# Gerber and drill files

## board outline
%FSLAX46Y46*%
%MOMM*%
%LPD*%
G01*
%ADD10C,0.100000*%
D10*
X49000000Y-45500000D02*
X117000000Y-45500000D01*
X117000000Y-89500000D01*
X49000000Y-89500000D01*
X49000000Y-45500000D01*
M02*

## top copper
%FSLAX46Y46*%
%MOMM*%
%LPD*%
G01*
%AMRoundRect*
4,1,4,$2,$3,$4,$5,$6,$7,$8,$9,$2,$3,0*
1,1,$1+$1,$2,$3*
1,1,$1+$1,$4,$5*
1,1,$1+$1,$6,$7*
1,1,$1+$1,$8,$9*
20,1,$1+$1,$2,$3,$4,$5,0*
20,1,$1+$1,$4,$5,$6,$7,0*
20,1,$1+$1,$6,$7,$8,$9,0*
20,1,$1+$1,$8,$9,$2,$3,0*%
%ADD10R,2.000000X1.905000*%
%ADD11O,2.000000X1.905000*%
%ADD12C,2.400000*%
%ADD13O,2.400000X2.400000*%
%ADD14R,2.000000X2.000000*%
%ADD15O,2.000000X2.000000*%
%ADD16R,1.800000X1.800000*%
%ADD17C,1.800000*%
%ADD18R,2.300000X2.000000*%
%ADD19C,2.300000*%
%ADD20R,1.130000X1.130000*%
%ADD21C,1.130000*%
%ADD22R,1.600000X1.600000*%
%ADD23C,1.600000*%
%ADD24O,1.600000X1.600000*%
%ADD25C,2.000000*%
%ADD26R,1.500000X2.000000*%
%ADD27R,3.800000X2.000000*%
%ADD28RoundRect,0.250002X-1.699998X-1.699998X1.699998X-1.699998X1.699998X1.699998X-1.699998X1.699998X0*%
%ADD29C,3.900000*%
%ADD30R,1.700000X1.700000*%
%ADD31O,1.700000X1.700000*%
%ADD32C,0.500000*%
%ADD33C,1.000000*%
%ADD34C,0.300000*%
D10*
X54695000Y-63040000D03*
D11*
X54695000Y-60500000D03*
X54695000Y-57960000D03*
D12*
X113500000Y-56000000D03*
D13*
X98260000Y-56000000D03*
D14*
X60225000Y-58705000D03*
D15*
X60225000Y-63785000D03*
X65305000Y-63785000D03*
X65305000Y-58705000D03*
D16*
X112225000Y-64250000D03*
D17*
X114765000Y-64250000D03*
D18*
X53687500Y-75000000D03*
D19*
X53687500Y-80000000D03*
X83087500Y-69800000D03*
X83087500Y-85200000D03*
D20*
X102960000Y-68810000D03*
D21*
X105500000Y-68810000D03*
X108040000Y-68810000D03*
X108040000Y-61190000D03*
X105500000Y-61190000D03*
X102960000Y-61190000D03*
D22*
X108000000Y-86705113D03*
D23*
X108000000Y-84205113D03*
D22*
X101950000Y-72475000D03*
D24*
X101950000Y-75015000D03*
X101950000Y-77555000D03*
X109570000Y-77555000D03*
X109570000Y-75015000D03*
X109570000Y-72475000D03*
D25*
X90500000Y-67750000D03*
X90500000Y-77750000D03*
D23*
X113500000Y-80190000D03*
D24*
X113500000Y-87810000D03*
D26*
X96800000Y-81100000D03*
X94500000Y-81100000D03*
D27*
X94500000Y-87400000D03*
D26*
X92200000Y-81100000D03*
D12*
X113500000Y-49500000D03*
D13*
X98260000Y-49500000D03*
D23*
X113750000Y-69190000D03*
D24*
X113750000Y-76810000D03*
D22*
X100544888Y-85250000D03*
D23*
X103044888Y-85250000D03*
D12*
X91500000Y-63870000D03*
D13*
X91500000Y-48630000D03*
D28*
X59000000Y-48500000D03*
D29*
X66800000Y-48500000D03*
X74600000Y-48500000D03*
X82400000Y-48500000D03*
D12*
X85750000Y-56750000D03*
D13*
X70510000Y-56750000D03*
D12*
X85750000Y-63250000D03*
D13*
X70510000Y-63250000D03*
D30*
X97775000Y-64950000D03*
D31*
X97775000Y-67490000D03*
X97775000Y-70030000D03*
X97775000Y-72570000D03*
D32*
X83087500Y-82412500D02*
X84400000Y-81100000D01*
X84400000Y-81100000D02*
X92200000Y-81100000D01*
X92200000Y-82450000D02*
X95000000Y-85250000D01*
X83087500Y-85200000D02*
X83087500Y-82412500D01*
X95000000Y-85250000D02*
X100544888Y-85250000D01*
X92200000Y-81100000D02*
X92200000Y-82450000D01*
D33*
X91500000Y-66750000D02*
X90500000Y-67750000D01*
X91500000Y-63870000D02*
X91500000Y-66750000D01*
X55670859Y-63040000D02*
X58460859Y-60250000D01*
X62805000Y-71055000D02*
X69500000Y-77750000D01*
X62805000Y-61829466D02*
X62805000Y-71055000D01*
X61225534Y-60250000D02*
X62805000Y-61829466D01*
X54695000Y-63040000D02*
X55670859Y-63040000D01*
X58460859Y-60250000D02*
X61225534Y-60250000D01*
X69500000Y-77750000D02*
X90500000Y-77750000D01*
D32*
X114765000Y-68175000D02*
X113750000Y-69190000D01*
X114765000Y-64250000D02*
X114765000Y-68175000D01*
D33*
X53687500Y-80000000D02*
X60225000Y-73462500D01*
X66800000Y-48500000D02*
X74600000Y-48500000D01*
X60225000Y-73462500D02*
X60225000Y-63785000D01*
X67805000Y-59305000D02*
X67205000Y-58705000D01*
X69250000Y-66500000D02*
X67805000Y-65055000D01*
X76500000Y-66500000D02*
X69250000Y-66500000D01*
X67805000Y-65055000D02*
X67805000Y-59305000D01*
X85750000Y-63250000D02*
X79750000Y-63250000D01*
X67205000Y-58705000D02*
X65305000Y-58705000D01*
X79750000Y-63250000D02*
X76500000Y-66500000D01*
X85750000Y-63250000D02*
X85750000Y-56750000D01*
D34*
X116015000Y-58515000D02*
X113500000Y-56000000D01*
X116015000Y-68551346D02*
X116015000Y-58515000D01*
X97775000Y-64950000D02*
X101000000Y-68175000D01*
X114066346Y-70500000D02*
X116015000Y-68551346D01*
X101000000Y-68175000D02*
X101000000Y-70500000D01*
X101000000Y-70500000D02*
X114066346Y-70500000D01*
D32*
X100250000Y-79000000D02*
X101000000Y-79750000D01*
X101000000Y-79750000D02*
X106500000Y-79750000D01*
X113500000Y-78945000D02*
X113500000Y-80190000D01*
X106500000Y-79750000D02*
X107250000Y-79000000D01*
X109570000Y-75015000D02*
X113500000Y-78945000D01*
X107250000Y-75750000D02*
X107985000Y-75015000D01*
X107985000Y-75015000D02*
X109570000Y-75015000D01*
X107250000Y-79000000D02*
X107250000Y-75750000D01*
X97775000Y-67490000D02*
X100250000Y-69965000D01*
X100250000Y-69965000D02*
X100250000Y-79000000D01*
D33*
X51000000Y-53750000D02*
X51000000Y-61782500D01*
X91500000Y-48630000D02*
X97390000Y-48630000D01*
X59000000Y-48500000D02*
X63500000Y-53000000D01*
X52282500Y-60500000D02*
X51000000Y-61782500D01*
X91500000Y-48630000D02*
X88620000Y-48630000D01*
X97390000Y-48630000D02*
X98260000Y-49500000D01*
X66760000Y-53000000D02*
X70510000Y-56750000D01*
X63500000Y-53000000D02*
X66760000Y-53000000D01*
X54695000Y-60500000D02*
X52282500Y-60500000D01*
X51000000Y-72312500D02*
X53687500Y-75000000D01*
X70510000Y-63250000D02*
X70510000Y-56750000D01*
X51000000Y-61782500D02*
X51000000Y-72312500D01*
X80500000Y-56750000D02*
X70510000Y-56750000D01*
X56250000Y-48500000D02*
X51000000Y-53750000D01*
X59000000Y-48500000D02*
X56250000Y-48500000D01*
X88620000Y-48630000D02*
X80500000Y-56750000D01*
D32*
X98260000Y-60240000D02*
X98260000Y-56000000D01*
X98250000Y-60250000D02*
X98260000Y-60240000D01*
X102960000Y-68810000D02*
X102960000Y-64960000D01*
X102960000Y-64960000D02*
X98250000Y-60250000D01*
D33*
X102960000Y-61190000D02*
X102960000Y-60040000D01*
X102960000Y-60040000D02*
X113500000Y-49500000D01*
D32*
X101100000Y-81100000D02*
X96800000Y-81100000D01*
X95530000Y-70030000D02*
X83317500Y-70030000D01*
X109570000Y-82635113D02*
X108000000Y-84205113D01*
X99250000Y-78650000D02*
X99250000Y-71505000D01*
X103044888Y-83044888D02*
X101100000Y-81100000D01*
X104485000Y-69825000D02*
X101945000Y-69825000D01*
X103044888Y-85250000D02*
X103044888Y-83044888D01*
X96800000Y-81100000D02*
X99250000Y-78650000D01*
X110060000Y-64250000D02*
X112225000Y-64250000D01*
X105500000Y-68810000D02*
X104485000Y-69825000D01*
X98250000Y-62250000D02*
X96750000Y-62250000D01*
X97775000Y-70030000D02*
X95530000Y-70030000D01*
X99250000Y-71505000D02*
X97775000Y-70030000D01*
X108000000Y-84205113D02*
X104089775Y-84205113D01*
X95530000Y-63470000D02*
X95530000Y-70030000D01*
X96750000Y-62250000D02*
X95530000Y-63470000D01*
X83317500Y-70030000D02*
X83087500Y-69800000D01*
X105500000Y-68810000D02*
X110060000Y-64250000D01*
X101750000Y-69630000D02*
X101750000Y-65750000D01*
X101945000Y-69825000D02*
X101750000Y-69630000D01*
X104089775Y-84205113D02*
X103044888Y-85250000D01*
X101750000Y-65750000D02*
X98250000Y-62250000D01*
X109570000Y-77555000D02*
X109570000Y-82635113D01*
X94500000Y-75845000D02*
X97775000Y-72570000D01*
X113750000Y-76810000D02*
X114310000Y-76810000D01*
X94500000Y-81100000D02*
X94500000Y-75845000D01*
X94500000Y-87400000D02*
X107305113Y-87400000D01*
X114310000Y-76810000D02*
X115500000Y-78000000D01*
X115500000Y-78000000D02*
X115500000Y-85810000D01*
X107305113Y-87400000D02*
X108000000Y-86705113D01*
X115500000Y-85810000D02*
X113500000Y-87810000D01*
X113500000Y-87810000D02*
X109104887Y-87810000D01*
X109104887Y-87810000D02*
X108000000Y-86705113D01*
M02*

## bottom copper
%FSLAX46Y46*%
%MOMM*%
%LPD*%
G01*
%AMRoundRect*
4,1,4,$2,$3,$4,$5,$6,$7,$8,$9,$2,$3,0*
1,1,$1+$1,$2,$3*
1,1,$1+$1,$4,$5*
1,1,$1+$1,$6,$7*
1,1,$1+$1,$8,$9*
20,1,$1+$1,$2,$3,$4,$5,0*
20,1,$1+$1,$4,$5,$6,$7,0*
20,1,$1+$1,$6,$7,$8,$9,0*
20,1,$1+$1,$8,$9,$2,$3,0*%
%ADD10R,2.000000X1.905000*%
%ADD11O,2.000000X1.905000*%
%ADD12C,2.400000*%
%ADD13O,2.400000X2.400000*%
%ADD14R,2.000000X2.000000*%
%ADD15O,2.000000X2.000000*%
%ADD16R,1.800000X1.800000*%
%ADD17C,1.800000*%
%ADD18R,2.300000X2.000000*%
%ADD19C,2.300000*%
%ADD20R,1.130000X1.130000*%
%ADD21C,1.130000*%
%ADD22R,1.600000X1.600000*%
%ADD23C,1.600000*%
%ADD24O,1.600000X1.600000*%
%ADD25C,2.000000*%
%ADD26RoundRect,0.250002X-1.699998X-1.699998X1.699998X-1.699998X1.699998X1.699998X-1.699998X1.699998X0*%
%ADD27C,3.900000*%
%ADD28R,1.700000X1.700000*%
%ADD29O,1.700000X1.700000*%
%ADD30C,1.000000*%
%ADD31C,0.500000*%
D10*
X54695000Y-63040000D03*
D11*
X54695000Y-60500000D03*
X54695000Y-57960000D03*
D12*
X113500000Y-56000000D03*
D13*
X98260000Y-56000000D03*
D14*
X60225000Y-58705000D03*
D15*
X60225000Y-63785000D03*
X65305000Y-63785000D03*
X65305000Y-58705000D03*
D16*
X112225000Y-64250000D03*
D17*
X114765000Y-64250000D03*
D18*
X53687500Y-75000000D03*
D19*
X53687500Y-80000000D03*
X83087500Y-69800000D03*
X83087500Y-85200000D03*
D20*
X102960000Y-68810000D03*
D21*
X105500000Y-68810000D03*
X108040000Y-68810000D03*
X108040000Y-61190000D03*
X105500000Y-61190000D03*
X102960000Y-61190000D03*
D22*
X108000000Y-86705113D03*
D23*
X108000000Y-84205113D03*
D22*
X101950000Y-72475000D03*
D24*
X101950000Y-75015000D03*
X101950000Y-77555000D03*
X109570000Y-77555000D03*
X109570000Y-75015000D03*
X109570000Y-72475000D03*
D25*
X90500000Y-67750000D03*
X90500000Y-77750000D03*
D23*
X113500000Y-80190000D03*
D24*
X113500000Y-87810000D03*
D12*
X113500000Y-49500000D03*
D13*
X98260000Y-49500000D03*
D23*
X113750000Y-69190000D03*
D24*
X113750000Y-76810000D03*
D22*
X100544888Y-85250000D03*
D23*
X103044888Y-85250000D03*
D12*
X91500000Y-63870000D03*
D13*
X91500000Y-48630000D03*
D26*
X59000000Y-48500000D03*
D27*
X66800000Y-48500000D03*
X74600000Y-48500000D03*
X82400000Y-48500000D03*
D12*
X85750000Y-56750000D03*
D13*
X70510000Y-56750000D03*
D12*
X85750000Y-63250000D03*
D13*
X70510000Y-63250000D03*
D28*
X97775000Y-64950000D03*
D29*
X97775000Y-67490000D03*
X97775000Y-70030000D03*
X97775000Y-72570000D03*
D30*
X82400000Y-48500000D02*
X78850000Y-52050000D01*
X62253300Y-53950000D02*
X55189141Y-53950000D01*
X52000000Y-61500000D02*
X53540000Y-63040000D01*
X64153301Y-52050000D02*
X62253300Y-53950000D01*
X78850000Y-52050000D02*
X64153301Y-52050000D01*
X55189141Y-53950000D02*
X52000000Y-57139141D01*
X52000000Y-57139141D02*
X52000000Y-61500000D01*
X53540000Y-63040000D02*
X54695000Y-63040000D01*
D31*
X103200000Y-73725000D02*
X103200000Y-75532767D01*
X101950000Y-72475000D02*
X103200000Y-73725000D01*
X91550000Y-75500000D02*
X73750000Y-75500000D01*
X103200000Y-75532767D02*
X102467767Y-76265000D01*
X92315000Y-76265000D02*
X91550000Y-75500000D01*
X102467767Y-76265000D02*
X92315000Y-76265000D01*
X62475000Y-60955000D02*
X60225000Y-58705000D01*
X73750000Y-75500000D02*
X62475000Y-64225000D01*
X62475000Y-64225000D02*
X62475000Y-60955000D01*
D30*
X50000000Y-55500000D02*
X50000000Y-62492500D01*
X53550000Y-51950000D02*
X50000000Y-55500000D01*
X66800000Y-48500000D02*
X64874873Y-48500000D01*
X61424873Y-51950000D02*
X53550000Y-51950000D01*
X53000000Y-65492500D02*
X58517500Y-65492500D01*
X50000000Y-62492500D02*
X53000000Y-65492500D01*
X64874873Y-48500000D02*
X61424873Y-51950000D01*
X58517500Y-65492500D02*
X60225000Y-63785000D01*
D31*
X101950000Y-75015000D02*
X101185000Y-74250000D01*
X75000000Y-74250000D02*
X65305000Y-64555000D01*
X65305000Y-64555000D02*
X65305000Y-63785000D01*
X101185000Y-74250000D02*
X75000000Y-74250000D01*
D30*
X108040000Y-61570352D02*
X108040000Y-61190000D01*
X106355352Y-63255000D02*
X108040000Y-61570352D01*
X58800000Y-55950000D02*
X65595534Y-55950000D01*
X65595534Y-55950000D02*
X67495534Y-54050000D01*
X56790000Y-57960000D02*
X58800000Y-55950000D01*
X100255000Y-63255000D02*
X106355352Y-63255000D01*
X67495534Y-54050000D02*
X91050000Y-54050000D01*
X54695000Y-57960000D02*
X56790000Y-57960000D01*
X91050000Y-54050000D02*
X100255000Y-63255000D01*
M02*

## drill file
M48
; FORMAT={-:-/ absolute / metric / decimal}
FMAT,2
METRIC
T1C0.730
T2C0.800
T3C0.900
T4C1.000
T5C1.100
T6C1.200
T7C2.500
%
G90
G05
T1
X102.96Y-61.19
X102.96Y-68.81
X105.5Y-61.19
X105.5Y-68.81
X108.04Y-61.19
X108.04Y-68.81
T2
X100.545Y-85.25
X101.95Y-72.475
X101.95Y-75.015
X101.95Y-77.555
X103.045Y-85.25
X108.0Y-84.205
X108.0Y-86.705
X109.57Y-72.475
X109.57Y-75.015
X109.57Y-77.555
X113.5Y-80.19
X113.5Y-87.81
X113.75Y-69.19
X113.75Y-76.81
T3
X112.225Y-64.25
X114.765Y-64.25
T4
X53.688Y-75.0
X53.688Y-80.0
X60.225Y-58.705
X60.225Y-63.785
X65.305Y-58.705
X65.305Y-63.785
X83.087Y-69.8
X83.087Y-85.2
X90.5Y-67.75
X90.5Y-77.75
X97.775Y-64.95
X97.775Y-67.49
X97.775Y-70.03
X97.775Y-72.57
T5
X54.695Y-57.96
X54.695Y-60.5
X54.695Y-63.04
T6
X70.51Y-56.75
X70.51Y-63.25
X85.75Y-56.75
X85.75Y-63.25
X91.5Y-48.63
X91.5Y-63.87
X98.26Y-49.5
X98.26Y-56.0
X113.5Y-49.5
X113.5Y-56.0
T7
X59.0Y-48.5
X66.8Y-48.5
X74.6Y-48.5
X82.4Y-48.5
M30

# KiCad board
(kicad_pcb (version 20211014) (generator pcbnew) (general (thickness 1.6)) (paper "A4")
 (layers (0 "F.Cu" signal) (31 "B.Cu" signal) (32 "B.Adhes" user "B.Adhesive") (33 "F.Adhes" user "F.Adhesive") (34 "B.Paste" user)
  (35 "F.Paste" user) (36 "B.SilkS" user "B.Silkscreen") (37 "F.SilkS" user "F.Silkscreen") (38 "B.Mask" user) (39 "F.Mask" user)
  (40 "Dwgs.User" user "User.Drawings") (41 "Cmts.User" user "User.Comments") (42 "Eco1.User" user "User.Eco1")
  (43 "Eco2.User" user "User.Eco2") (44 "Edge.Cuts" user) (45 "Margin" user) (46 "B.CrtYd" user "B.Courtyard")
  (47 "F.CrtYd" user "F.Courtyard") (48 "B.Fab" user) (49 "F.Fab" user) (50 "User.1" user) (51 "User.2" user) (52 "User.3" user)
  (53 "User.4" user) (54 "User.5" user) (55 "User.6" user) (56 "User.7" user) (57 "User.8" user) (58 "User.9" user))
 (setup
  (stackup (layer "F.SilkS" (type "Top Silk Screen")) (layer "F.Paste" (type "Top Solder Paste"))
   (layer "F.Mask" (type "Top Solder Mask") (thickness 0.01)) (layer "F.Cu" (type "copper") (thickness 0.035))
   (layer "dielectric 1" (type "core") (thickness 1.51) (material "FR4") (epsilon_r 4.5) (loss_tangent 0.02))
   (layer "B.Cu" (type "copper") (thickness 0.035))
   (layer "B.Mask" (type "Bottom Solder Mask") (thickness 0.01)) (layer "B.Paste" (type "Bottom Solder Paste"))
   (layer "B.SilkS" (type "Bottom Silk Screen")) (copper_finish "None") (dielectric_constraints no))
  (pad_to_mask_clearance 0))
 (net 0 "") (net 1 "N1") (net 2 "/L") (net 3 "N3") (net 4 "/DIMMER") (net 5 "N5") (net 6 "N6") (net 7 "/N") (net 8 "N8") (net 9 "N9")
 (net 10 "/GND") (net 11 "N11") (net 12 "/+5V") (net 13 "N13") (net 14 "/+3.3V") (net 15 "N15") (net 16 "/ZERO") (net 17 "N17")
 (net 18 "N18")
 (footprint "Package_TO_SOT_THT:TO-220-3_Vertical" (layer "F.Cu") (at 54.695 63.04 90)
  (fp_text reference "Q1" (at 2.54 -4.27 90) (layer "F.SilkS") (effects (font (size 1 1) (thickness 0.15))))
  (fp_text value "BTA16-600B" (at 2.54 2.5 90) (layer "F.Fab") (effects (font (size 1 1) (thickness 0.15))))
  (pad "1" thru_hole rect (at 0 0 90) (size 1.905 2) (drill 1.1) (layers *.Cu *.Mask) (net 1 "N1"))
  (pad "2" thru_hole oval (at 2.54 0 90) (size 1.905 2) (drill 1.1) (layers *.Cu *.Mask) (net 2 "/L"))
  (pad "3" thru_hole oval (at 5.08 0 90) (size 1.905 2) (drill 1.1) (layers *.Cu *.Mask) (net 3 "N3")))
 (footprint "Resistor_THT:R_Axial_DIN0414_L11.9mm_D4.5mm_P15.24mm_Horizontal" (layer "F.Cu") (at 113.5 56 180)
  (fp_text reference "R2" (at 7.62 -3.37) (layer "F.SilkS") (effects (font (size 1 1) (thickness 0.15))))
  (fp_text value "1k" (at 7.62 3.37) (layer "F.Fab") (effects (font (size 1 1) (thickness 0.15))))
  (pad "1" thru_hole circle (at 0 0 180) (size 2.4 2.4) (drill 1.2) (layers *.Cu *.Mask) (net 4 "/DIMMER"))
  (pad "2" thru_hole oval (at 15.24 0 180) (size 2.4 2.4) (drill 1.2) (layers *.Cu *.Mask) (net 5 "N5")))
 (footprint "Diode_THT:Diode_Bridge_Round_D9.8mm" (layer "F.Cu") (at 60.225 58.705)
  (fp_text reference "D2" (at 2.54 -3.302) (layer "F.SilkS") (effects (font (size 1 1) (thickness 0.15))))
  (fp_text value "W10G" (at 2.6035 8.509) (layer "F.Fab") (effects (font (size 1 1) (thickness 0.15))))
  (pad "1" thru_hole rect (at 0 0) (size 2 2) (drill 1) (layers *.Cu *.Mask) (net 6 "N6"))
  (pad "2" thru_hole oval (at 0 5.08) (size 2 2) (drill 1) (layers *.Cu *.Mask) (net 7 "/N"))
  (pad "3" thru_hole oval (at 5.08 5.08) (size 2 2) (drill 1) (layers *.Cu *.Mask) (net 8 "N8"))
  (pad "4" thru_hole oval (at 5.08 0) (size 2 2) (drill 1) (layers *.Cu *.Mask) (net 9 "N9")))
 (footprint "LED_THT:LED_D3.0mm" (layer "F.Cu") (at 112.225 64.25)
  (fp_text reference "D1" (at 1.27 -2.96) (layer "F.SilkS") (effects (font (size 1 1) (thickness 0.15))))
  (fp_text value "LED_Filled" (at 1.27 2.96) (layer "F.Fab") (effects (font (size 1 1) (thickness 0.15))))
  (pad "1" thru_hole rect (at 0 0) (size 1.8 1.8) (drill 0.9) (layers *.Cu *.Mask) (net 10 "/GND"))
  (pad "2" thru_hole circle (at 2.54 0) (size 1.8 1.8) (drill 0.9) (layers *.Cu *.Mask) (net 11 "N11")))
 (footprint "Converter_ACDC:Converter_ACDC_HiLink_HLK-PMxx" (layer "F.Cu") (at 53.6875 75)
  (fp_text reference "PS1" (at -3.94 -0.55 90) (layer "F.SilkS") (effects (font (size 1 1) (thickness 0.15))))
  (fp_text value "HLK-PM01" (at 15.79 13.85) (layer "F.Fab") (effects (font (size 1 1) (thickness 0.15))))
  (pad "1" thru_hole rect (at 0 0) (size 2.3 2) (drill 1) (layers *.Cu *.Mask) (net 2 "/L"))
  (pad "2" thru_hole circle (at 0 5) (size 2.3 2.3) (drill 1) (layers *.Cu *.Mask) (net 7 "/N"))
  (pad "3" thru_hole circle (at 29.4 -5.2) (size 2.3 2.3) (drill 1) (layers *.Cu *.Mask) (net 10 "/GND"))
  (pad "4" thru_hole circle (at 29.4 10.2) (size 2.3 2.3) (drill 1) (layers *.Cu *.Mask) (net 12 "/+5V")))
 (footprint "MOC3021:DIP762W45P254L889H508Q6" (layer "F.Cu") (at 105.5 65 90)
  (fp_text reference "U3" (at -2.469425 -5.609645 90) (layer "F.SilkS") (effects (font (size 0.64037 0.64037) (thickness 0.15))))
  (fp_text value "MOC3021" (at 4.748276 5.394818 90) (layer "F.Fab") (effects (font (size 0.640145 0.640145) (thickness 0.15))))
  (pad "1" thru_hole rect locked (at -3.81 -2.54 90) (size 1.13 1.13) (drill 0.73) (layers *.Cu *.Mask) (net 5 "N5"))
  (pad "2" thru_hole circle locked (at -3.81 0 90) (size 1.13 1.13) (drill 0.73) (layers *.Cu *.Mask) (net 10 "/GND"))
  (pad "3" thru_hole circle locked (at -3.81 2.54 90) (size 1.13 1.13) (drill 0.73) (layers *.Cu *.Mask))
  (pad "4" thru_hole circle locked (at 3.81 2.54 90) (size 1.13 1.13) (drill 0.73) (layers *.Cu *.Mask) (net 3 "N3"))
  (pad "5" thru_hole circle locked (at 3.81 0 90) (size 1.13 1.13) (drill 0.73) (layers *.Cu *.Mask))
  (pad "6" thru_hole circle locked (at 3.81 -2.54 90) (size 1.13 1.13) (drill 0.73) (layers *.Cu *.Mask) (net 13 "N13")))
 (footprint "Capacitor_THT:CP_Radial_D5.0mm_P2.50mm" (layer "F.Cu") (at 108 86.705113 90)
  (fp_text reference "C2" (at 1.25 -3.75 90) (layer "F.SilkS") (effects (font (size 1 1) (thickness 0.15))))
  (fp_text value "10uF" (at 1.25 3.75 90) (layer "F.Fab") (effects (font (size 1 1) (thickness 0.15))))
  (pad "1" thru_hole rect (at 0 0 90) (size 1.6 1.6) (drill 0.8) (layers *.Cu *.Mask) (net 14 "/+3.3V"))
  (pad "2" thru_hole circle (at 2.5 0 90) (size 1.6 1.6) (drill 0.8) (layers *.Cu *.Mask) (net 10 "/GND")))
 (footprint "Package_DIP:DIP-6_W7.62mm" (layer "F.Cu") (at 101.95 72.475)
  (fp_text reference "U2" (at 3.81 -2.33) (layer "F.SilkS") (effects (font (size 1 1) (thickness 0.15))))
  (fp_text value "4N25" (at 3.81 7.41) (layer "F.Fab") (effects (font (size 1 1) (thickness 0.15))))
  (pad "1" thru_hole rect (at 0 0) (size 1.6 1.6) (drill 0.8) (layers *.Cu *.Mask) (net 6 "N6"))
  (pad "2" thru_hole oval (at 0 2.54) (size 1.6 1.6) (drill 0.8) (layers *.Cu *.Mask) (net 8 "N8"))
  (pad "3" thru_hole oval (at 0 5.08) (size 1.6 1.6) (drill 0.8) (layers *.Cu *.Mask) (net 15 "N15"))
  (pad "4" thru_hole oval (at 7.62 5.08) (size 1.6 1.6) (drill 0.8) (layers *.Cu *.Mask) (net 10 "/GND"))
  (pad "5" thru_hole oval (at 7.62 2.54) (size 1.6 1.6) (drill 0.8) (layers *.Cu *.Mask) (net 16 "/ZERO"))
  (pad "6" thru_hole oval (at 7.62 0) (size 1.6 1.6) (drill 0.8) (layers *.Cu *.Mask) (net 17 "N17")))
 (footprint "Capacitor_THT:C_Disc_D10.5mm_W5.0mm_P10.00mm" (layer "F.Cu") (at 90.5 67.75 -90)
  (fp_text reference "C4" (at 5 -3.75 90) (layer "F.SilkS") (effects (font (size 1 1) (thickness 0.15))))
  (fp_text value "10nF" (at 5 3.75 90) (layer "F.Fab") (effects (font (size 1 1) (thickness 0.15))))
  (pad "1" thru_hole circle (at 0 0 270) (size 2 2) (drill 1) (layers *.Cu *.Mask) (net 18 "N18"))
  (pad "2" thru_hole circle (at 10 0 270) (size 2 2) (drill 1) (layers *.Cu *.Mask) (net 1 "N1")))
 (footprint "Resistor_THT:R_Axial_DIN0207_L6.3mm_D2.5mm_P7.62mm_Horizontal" (layer "F.Cu") (at 113.5 80.19 -90)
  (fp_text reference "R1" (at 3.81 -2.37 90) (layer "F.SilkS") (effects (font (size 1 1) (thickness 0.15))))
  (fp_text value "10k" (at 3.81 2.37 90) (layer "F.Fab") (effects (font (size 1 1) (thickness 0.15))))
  (pad "1" thru_hole circle (at 0 0 270) (size 1.6 1.6) (drill 0.8) (layers *.Cu *.Mask) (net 16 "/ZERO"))
  (pad "2" thru_hole oval (at 7.62 0 270) (size 1.6 1.6) (drill 0.8) (layers *.Cu *.Mask) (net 14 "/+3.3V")))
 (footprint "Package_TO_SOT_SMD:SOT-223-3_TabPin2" (layer "F.Cu") (at 94.5 84.25 -90)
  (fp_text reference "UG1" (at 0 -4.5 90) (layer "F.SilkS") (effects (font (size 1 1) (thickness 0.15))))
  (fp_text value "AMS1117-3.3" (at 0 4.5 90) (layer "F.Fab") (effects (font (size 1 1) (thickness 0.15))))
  (pad "1" smd rect (at -3.15 -2.3 270) (size 2 1.5) (layers "F.Cu" "F.Paste" "F.Mask") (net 10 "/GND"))
  (pad "2" smd rect (at -3.15 0 270) (size 2 1.5) (layers "F.Cu" "F.Paste" "F.Mask") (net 14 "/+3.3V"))
  (pad "2" smd rect (at 3.15 0 270) (size 2 3.8) (layers "F.Cu" "F.Paste" "F.Mask") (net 14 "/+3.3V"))
  (pad "3" smd rect (at -3.15 2.3 270) (size 2 1.5) (layers "F.Cu" "F.Paste" "F.Mask") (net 12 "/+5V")))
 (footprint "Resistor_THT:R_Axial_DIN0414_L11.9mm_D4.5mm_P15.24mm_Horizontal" (layer "F.Cu") (at 113.5 49.5 180)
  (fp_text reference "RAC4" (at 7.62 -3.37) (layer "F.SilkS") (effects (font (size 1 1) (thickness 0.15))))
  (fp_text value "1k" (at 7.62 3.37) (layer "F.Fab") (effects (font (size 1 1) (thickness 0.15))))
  (pad "1" thru_hole circle (at 0 0 180) (size 2.4 2.4) (drill 1.2) (layers *.Cu *.Mask) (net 13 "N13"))
  (pad "2" thru_hole oval (at 15.24 0 180) (size 2.4 2.4) (drill 1.2) (layers *.Cu *.Mask) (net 2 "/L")))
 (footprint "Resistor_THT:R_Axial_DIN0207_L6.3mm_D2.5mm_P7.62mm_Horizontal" (layer "F.Cu") (at 113.75 69.19 -90)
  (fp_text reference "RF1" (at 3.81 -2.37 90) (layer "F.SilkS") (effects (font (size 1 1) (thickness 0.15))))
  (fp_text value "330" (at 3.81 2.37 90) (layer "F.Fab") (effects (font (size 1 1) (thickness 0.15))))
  (pad "1" thru_hole circle (at 0 0 270) (size 1.6 1.6) (drill 0.8) (layers *.Cu *.Mask) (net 11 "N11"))
  (pad "2" thru_hole oval (at 7.62 0 270) (size 1.6 1.6) (drill 0.8) (layers *.Cu *.Mask) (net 14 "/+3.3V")))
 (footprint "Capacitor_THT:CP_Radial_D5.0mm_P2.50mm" (layer "F.Cu") (at 100.544888 85.25)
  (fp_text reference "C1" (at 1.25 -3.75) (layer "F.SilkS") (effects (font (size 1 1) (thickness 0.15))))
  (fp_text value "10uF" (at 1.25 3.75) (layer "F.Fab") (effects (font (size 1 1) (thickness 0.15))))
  (pad "1" thru_hole rect (at 0 0) (size 1.6 1.6) (drill 0.8) (layers *.Cu *.Mask) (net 12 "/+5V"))
  (pad "2" thru_hole circle (at 2.5 0) (size 1.6 1.6) (drill 0.8) (layers *.Cu *.Mask) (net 10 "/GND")))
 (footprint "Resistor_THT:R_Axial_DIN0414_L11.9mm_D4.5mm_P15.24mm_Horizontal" (layer "F.Cu") (at 91.5 63.87 90)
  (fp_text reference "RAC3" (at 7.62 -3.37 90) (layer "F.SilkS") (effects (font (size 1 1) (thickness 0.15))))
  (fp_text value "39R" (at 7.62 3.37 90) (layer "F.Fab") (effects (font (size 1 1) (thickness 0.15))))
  (pad "1" thru_hole circle (at 0 0 90) (size 2.4 2.4) (drill 1.2) (layers *.Cu *.Mask) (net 18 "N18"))
  (pad "2" thru_hole oval (at 15.24 0 90) (size 2.4 2.4) (drill 1.2) (layers *.Cu *.Mask) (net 2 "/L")))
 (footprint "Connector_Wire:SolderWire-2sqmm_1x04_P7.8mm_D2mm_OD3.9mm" (layer "F.Cu") (at 59 48.5)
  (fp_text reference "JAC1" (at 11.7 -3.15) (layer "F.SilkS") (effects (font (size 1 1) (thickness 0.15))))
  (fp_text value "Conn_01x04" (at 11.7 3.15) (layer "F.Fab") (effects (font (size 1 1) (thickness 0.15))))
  (pad "1" thru_hole roundrect (at 0 0) (size 3.9 3.9) (drill 2.5) (layers *.Cu *.Mask) (roundrect_rratio 0.064103) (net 2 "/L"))
  (pad "2" thru_hole circle (at 7.8 0) (size 3.9 3.9) (drill 2.5) (layers *.Cu *.Mask) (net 7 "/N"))
  (pad "3" thru_hole circle (at 15.6 0) (size 3.9 3.9) (drill 2.5) (layers *.Cu *.Mask) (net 7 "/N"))
  (pad "4" thru_hole circle (at 23.4 0) (size 3.9 3.9) (drill 2.5) (layers *.Cu *.Mask) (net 1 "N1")))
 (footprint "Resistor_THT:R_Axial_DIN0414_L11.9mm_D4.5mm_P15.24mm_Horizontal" (layer "F.Cu") (at 85.75 56.75 180)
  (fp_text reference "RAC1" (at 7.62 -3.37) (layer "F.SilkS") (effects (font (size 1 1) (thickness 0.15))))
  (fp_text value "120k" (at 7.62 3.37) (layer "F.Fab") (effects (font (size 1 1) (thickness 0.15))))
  (pad "1" thru_hole circle (at 0 0 180) (size 2.4 2.4) (drill 1.2) (layers *.Cu *.Mask) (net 9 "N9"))
  (pad "2" thru_hole oval (at 15.24 0 180) (size 2.4 2.4) (drill 1.2) (layers *.Cu *.Mask) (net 2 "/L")))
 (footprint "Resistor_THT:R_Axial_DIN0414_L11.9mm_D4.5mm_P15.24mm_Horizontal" (layer "F.Cu") (at 85.75 63.25 180)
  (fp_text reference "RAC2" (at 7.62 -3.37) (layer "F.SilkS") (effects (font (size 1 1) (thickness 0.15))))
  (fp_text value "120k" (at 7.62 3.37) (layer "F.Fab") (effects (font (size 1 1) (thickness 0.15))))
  (pad "1" thru_hole circle (at 0 0 180) (size 2.4 2.4) (drill 1.2) (layers *.Cu *.Mask) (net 9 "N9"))
  (pad "2" thru_hole oval (at 15.24 0 180) (size 2.4 2.4) (drill 1.2) (layers *.Cu *.Mask) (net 2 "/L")))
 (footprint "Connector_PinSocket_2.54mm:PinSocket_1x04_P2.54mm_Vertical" (layer "F.Cu") (at 97.775 64.95)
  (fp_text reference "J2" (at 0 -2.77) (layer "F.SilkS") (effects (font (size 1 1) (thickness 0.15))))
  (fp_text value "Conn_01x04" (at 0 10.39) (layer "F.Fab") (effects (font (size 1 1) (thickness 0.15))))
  (pad "1" thru_hole rect (at 0 0) (size 1.7 1.7) (drill 1) (layers *.Cu *.Mask) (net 4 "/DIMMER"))
  (pad "2" thru_hole oval (at 0 2.54) (size 1.7 1.7) (drill 1) (layers *.Cu *.Mask) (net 16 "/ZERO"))
  (pad "3" thru_hole oval (at 0 5.08) (size 1.7 1.7) (drill 1) (layers *.Cu *.Mask) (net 10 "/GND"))
  (pad "4" thru_hole oval (at 0 7.62) (size 1.7 1.7) (drill 1) (layers *.Cu *.Mask) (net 14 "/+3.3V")))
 (gr_rect (start 49 45.5) (end 117 89.5) (layer "Edge.Cuts") (width 0.1) (fill none))
 (segment (start 83.0875 82.4125) (end 84.4 81.1) (width 0.5) (layer "F.Cu") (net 12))
 (segment (start 84.4 81.1) (end 92.2 81.1) (width 0.5) (layer "F.Cu") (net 12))
 (segment (start 92.2 82.45) (end 95 85.25) (width 0.5) (layer "F.Cu") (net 12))
 (segment (start 83.0875 85.2) (end 83.0875 82.4125) (width 0.5) (layer "F.Cu") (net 12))
 (segment (start 95 85.25) (end 100.544888 85.25) (width 0.5) (layer "F.Cu") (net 12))
 (segment (start 92.2 81.1) (end 92.2 82.45) (width 0.5) (layer "F.Cu") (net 12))
 (segment (start 91.5 66.75) (end 90.5 67.75) (width 1) (layer "F.Cu") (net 18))
 (segment (start 91.5 63.87) (end 91.5 66.75) (width 1) (layer "F.Cu") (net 18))
 (segment (start 55.670859 63.04) (end 58.460859 60.25) (width 1) (layer "F.Cu") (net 1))
 (segment (start 62.805 71.055) (end 69.5 77.75) (width 1) (layer "F.Cu") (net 1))
 (segment (start 62.805 61.829466) (end 62.805 71.055) (width 1) (layer "F.Cu") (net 1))
 (segment (start 61.225534 60.25) (end 62.805 61.829466) (width 1) (layer "F.Cu") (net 1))
 (segment (start 54.695 63.04) (end 55.670859 63.04) (width 1) (layer "F.Cu") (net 1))
 (segment (start 58.460859 60.25) (end 61.225534 60.25) (width 1) (layer "F.Cu") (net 1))
 (segment (start 69.5 77.75) (end 90.5 77.75) (width 1) (layer "F.Cu") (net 1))
 (segment (start 82.4 48.5) (end 78.85 52.05) (width 1) (layer "B.Cu") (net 1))
 (segment (start 62.2533 53.95) (end 55.189141 53.95) (width 1) (layer "B.Cu") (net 1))
 (segment (start 52 61.5) (end 53.54 63.04) (width 1) (layer "B.Cu") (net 1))
 (segment (start 64.153301 52.05) (end 62.2533 53.95) (width 1) (layer "B.Cu") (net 1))
 (segment (start 78.85 52.05) (end 64.153301 52.05) (width 1) (layer "B.Cu") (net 1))
 (segment (start 55.189141 53.95) (end 52 57.139141) (width 1) (layer "B.Cu") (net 1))
 (segment (start 52 57.139141) (end 52 61.5) (width 1) (layer "B.Cu") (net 1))
 (segment (start 53.54 63.04) (end 54.695 63.04) (width 1) (layer "B.Cu") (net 1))
 (segment (start 114.765 68.175) (end 113.75 69.19) (width 0.5) (layer "F.Cu") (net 11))
 (segment (start 114.765 64.25) (end 114.765 68.175) (width 0.5) (layer "F.Cu") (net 11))
 (segment (start 103.2 73.725) (end 103.2 75.532767) (width 0.5) (layer "B.Cu") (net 6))
 (segment (start 101.95 72.475) (end 103.2 73.725) (width 0.5) (layer "B.Cu") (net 6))
 (segment (start 91.55 75.5) (end 73.75 75.5) (width 0.5) (layer "B.Cu") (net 6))
 (segment (start 103.2 75.532767) (end 102.467767 76.265) (width 0.5) (layer "B.Cu") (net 6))
 (segment (start 92.315 76.265) (end 91.55 75.5) (width 0.5) (layer "B.Cu") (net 6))
 (segment (start 102.467767 76.265) (end 92.315 76.265) (width 0.5) (layer "B.Cu") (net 6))
 (segment (start 62.475 60.955) (end 60.225 58.705) (width 0.5) (layer "B.Cu") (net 6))
 (segment (start 73.75 75.5) (end 62.475 64.225) (width 0.5) (layer "B.Cu") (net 6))
 (segment (start 62.475 64.225) (end 62.475 60.955) (width 0.5) (layer "B.Cu") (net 6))
 (segment (start 53.6875 80) (end 60.225 73.4625) (width 1) (layer "F.Cu") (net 7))
 (segment (start 66.8 48.5) (end 74.6 48.5) (width 1) (layer "F.Cu") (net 7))
 (segment (start 60.225 73.4625) (end 60.225 63.785) (width 1) (layer "F.Cu") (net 7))
 (segment (start 50 55.5) (end 50 62.4925) (width 1) (layer "B.Cu") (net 7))
 (segment (start 53.55 51.95) (end 50 55.5) (width 1) (layer "B.Cu") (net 7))
 (segment (start 66.8 48.5) (end 64.874873 48.5) (width 1) (layer "B.Cu") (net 7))
 (segment (start 61.424873 51.95) (end 53.55 51.95) (width 1) (layer "B.Cu") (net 7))
 (segment (start 53 65.4925) (end 58.5175 65.4925) (width 1) (layer "B.Cu") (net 7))
 (segment (start 50 62.4925) (end 53 65.4925) (width 1) (layer "B.Cu") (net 7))
 (segment (start 64.874873 48.5) (end 61.424873 51.95) (width 1) (layer "B.Cu") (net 7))
 (segment (start 58.5175 65.4925) (end 60.225 63.785) (width 1) (layer "B.Cu") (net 7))
 (segment (start 101.95 75.015) (end 101.185 74.25) (width 0.5) (layer "B.Cu") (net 8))
 (segment (start 75 74.25) (end 65.305 64.555) (width 0.5) (layer "B.Cu") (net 8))
 (segment (start 65.305 64.555) (end 65.305 63.785) (width 0.5) (layer "B.Cu") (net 8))
 (segment (start 101.185 74.25) (end 75 74.25) (width 0.5) (layer "B.Cu") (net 8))
 (segment (start 67.805 59.305) (end 67.205 58.705) (width 1) (layer "F.Cu") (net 9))
 (segment (start 69.25 66.5) (end 67.805 65.055) (width 1) (layer "F.Cu") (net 9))
 (segment (start 76.5 66.5) (end 69.25 66.5) (width 1) (layer "F.Cu") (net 9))
 (segment (start 67.805 65.055) (end 67.805 59.305) (width 1) (layer "F.Cu") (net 9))
 (segment (start 85.75 63.25) (end 79.75 63.25) (width 1) (layer "F.Cu") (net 9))
 (segment (start 67.205 58.705) (end 65.305 58.705) (width 1) (layer "F.Cu") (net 9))
 (segment (start 79.75 63.25) (end 76.5 66.5) (width 1) (layer "F.Cu") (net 9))
 (segment (start 85.75 63.25) (end 85.75 56.75) (width 1) (layer "F.Cu") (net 9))
 (segment (start 116.015 58.515) (end 113.5 56) (width 0.3) (layer "F.Cu") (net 4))
 (segment (start 116.015 68.551346) (end 116.015 58.515) (width 0.3) (layer "F.Cu") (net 4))
 (segment (start 97.775 64.95) (end 101 68.175) (width 0.3) (layer "F.Cu") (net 4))
 (segment (start 114.066346 70.5) (end 116.015 68.551346) (width 0.3) (layer "F.Cu") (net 4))
 (segment (start 101 68.175) (end 101 70.5) (width 0.3) (layer "F.Cu") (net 4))
 (segment (start 101 70.5) (end 114.066346 70.5) (width 0.3) (layer "F.Cu") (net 4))
 (segment (start 100.25 79) (end 101 79.75) (width 0.5) (layer "F.Cu") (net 16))
 (segment (start 101 79.75) (end 106.5 79.75) (width 0.5) (layer "F.Cu") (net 16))
 (segment (start 113.5 78.945) (end 113.5 80.19) (width 0.5) (layer "F.Cu") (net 16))
 (segment (start 106.5 79.75) (end 107.25 79) (width 0.5) (layer "F.Cu") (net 16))
 (segment (start 109.57 75.015) (end 113.5 78.945) (width 0.5) (layer "F.Cu") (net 16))
 (segment (start 107.25 75.75) (end 107.985 75.015) (width 0.5) (layer "F.Cu") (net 16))
 (segment (start 107.985 75.015) (end 109.57 75.015) (width 0.5) (layer "F.Cu") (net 16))
 (segment (start 107.25 79) (end 107.25 75.75) (width 0.5) (layer "F.Cu") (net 16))
 (segment (start 97.775 67.49) (end 100.25 69.965) (width 0.5) (layer "F.Cu") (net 16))
 (segment (start 100.25 69.965) (end 100.25 79) (width 0.5) (layer "F.Cu") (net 16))
 (segment (start 51 53.75) (end 51 61.7825) (width 1) (layer "F.Cu") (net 2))
 (segment (start 91.5 48.63) (end 97.39 48.63) (width 1) (layer "F.Cu") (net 2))
 (segment (start 59 48.5) (end 63.5 53) (width 1) (layer "F.Cu") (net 2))
 (segment (start 52.2825 60.5) (end 51 61.7825) (width 1) (layer "F.Cu") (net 2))
 (segment (start 91.5 48.63) (end 88.62 48.63) (width 1) (layer "F.Cu") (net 2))
 (segment (start 97.39 48.63) (end 98.26 49.5) (width 1) (layer "F.Cu") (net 2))
 (segment (start 66.76 53) (end 70.51 56.75) (width 1) (layer "F.Cu") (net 2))
 (segment (start 63.5 53) (end 66.76 53) (width 1) (layer "F.Cu") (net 2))
 (segment (start 54.695 60.5) (end 52.2825 60.5) (width 1) (layer "F.Cu") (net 2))
 (segment (start 51 72.3125) (end 53.6875 75) (width 1) (layer "F.Cu") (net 2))
 (segment (start 70.51 63.25) (end 70.51 56.75) (width 1) (layer "F.Cu") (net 2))
 (segment (start 51 61.7825) (end 51 72.3125) (width 1) (layer "F.Cu") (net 2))
 (segment (start 80.5 56.75) (end 70.51 56.75) (width 1) (layer "F.Cu") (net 2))
 (segment (start 56.25 48.5) (end 51 53.75) (width 1) (layer "F.Cu") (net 2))
 (segment (start 59 48.5) (end 56.25 48.5) (width 1) (layer "F.Cu") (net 2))
 (segment (start 88.62 48.63) (end 80.5 56.75) (width 1) (layer "F.Cu") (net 2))
 (segment (start 108.04 61.570352) (end 108.04 61.19) (width 1) (layer "B.Cu") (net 3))
 (segment (start 106.355352 63.255) (end 108.04 61.570352) (width 1) (layer "B.Cu") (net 3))
 (segment (start 58.8 55.95) (end 65.595534 55.95) (width 1) (layer "B.Cu") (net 3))
 (segment (start 65.595534 55.95) (end 67.495534 54.05) (width 1) (layer "B.Cu") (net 3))
 (segment (start 56.79 57.96) (end 58.8 55.95) (width 1) (layer "B.Cu") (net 3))
 (segment (start 100.255 63.255) (end 106.355352 63.255) (width 1) (layer "B.Cu") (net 3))
 (segment (start 67.495534 54.05) (end 91.05 54.05) (width 1) (layer "B.Cu") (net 3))
 (segment (start 54.695 57.96) (end 56.79 57.96) (width 1) (layer "B.Cu") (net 3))
 (segment (start 91.05 54.05) (end 100.255 63.255) (width 1) (layer "B.Cu") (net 3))
 (segment (start 98.26 60.24) (end 98.26 56) (width 0.5) (layer "F.Cu") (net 5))
 (segment (start 98.25 60.25) (end 98.26 60.24) (width 0.5) (layer "F.Cu") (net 5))
 (segment (start 102.96 68.81) (end 102.96 64.96) (width 0.5) (layer "F.Cu") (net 5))
 (segment (start 102.96 64.96) (end 98.25 60.25) (width 0.5) (layer "F.Cu") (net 5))
 (segment (start 102.96 61.19) (end 102.96 60.04) (width 1) (layer "F.Cu") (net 13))
 (segment (start 102.96 60.04) (end 113.5 49.5) (width 1) (layer "F.Cu") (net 13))
 (segment (start 101.1 81.1) (end 96.8 81.1) (width 0.5) (layer "F.Cu") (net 10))
 (segment (start 95.53 70.03) (end 83.3175 70.03) (width 0.5) (layer "F.Cu") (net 10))
 (segment (start 109.57 82.635113) (end 108 84.205113) (width 0.5) (layer "F.Cu") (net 10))
 (segment (start 99.25 78.65) (end 99.25 71.505) (width 0.5) (layer "F.Cu") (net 10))
 (segment (start 103.044888 83.044888) (end 101.1 81.1) (width 0.5) (layer "F.Cu") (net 10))
 (segment (start 104.485 69.825) (end 101.945 69.825) (width 0.5) (layer "F.Cu") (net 10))
 (segment (start 103.044888 85.25) (end 103.044888 83.044888) (width 0.5) (layer "F.Cu") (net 10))
 (segment (start 96.8 81.1) (end 99.25 78.65) (width 0.5) (layer "F.Cu") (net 10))
 (segment (start 110.06 64.25) (end 112.225 64.25) (width 0.5) (layer "F.Cu") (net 10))
 (segment (start 105.5 68.81) (end 104.485 69.825) (width 0.5) (layer "F.Cu") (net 10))
 (segment (start 98.25 62.25) (end 96.75 62.25) (width 0.5) (layer "F.Cu") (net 10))
 (segment (start 97.775 70.03) (end 95.53 70.03) (width 0.5) (layer "F.Cu") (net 10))
 (segment (start 99.25 71.505) (end 97.775 70.03) (width 0.5) (layer "F.Cu") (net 10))
 (segment (start 108 84.205113) (end 104.089775 84.205113) (width 0.5) (layer "F.Cu") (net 10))
 (segment (start 95.53 63.47) (end 95.53 70.03) (width 0.5) (layer "F.Cu") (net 10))
 (segment (start 96.75 62.25) (end 95.53 63.47) (width 0.5) (layer "F.Cu") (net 10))
 (segment (start 83.3175 70.03) (end 83.0875 69.8) (width 0.5) (layer "F.Cu") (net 10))
 (segment (start 105.5 68.81) (end 110.06 64.25) (width 0.5) (layer "F.Cu") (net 10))
 (segment (start 101.75 69.63) (end 101.75 65.75) (width 0.5) (layer "F.Cu") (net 10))
 (segment (start 101.945 69.825) (end 101.75 69.63) (width 0.5) (layer "F.Cu") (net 10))
 (segment (start 104.089775 84.205113) (end 103.044888 85.25) (width 0.5) (layer "F.Cu") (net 10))
 (segment (start 101.75 65.75) (end 98.25 62.25) (width 0.5) (layer "F.Cu") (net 10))
 (segment (start 109.57 77.555) (end 109.57 82.635113) (width 0.5) (layer "F.Cu") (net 10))
 (segment (start 94.5 75.845) (end 97.775 72.57) (width 0.5) (layer "F.Cu") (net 14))
 (segment (start 113.75 76.81) (end 114.31 76.81) (width 0.5) (layer "F.Cu") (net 14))
 (segment (start 94.5 81.1) (end 94.5 75.845) (width 0.5) (layer "F.Cu") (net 14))
 (segment (start 94.5 87.4) (end 107.305113 87.4) (width 0.5) (layer "F.Cu") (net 14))
 (segment (start 114.31 76.81) (end 115.5 78) (width 0.5) (layer "F.Cu") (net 14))
 (segment (start 115.5 78) (end 115.5 85.81) (width 0.5) (layer "F.Cu") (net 14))
 (segment (start 107.305113 87.4) (end 108 86.705113) (width 0.5) (layer "F.Cu") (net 14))
 (segment (start 115.5 85.81) (end 113.5 87.81) (width 0.5) (layer "F.Cu") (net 14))
 (segment (start 113.5 87.81) (end 109.104887 87.81) (width 0.5) (layer "F.Cu") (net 14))
 (segment (start 109.104887 87.81) (end 108 86.705113) (width 0.5) (layer "F.Cu") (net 14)))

